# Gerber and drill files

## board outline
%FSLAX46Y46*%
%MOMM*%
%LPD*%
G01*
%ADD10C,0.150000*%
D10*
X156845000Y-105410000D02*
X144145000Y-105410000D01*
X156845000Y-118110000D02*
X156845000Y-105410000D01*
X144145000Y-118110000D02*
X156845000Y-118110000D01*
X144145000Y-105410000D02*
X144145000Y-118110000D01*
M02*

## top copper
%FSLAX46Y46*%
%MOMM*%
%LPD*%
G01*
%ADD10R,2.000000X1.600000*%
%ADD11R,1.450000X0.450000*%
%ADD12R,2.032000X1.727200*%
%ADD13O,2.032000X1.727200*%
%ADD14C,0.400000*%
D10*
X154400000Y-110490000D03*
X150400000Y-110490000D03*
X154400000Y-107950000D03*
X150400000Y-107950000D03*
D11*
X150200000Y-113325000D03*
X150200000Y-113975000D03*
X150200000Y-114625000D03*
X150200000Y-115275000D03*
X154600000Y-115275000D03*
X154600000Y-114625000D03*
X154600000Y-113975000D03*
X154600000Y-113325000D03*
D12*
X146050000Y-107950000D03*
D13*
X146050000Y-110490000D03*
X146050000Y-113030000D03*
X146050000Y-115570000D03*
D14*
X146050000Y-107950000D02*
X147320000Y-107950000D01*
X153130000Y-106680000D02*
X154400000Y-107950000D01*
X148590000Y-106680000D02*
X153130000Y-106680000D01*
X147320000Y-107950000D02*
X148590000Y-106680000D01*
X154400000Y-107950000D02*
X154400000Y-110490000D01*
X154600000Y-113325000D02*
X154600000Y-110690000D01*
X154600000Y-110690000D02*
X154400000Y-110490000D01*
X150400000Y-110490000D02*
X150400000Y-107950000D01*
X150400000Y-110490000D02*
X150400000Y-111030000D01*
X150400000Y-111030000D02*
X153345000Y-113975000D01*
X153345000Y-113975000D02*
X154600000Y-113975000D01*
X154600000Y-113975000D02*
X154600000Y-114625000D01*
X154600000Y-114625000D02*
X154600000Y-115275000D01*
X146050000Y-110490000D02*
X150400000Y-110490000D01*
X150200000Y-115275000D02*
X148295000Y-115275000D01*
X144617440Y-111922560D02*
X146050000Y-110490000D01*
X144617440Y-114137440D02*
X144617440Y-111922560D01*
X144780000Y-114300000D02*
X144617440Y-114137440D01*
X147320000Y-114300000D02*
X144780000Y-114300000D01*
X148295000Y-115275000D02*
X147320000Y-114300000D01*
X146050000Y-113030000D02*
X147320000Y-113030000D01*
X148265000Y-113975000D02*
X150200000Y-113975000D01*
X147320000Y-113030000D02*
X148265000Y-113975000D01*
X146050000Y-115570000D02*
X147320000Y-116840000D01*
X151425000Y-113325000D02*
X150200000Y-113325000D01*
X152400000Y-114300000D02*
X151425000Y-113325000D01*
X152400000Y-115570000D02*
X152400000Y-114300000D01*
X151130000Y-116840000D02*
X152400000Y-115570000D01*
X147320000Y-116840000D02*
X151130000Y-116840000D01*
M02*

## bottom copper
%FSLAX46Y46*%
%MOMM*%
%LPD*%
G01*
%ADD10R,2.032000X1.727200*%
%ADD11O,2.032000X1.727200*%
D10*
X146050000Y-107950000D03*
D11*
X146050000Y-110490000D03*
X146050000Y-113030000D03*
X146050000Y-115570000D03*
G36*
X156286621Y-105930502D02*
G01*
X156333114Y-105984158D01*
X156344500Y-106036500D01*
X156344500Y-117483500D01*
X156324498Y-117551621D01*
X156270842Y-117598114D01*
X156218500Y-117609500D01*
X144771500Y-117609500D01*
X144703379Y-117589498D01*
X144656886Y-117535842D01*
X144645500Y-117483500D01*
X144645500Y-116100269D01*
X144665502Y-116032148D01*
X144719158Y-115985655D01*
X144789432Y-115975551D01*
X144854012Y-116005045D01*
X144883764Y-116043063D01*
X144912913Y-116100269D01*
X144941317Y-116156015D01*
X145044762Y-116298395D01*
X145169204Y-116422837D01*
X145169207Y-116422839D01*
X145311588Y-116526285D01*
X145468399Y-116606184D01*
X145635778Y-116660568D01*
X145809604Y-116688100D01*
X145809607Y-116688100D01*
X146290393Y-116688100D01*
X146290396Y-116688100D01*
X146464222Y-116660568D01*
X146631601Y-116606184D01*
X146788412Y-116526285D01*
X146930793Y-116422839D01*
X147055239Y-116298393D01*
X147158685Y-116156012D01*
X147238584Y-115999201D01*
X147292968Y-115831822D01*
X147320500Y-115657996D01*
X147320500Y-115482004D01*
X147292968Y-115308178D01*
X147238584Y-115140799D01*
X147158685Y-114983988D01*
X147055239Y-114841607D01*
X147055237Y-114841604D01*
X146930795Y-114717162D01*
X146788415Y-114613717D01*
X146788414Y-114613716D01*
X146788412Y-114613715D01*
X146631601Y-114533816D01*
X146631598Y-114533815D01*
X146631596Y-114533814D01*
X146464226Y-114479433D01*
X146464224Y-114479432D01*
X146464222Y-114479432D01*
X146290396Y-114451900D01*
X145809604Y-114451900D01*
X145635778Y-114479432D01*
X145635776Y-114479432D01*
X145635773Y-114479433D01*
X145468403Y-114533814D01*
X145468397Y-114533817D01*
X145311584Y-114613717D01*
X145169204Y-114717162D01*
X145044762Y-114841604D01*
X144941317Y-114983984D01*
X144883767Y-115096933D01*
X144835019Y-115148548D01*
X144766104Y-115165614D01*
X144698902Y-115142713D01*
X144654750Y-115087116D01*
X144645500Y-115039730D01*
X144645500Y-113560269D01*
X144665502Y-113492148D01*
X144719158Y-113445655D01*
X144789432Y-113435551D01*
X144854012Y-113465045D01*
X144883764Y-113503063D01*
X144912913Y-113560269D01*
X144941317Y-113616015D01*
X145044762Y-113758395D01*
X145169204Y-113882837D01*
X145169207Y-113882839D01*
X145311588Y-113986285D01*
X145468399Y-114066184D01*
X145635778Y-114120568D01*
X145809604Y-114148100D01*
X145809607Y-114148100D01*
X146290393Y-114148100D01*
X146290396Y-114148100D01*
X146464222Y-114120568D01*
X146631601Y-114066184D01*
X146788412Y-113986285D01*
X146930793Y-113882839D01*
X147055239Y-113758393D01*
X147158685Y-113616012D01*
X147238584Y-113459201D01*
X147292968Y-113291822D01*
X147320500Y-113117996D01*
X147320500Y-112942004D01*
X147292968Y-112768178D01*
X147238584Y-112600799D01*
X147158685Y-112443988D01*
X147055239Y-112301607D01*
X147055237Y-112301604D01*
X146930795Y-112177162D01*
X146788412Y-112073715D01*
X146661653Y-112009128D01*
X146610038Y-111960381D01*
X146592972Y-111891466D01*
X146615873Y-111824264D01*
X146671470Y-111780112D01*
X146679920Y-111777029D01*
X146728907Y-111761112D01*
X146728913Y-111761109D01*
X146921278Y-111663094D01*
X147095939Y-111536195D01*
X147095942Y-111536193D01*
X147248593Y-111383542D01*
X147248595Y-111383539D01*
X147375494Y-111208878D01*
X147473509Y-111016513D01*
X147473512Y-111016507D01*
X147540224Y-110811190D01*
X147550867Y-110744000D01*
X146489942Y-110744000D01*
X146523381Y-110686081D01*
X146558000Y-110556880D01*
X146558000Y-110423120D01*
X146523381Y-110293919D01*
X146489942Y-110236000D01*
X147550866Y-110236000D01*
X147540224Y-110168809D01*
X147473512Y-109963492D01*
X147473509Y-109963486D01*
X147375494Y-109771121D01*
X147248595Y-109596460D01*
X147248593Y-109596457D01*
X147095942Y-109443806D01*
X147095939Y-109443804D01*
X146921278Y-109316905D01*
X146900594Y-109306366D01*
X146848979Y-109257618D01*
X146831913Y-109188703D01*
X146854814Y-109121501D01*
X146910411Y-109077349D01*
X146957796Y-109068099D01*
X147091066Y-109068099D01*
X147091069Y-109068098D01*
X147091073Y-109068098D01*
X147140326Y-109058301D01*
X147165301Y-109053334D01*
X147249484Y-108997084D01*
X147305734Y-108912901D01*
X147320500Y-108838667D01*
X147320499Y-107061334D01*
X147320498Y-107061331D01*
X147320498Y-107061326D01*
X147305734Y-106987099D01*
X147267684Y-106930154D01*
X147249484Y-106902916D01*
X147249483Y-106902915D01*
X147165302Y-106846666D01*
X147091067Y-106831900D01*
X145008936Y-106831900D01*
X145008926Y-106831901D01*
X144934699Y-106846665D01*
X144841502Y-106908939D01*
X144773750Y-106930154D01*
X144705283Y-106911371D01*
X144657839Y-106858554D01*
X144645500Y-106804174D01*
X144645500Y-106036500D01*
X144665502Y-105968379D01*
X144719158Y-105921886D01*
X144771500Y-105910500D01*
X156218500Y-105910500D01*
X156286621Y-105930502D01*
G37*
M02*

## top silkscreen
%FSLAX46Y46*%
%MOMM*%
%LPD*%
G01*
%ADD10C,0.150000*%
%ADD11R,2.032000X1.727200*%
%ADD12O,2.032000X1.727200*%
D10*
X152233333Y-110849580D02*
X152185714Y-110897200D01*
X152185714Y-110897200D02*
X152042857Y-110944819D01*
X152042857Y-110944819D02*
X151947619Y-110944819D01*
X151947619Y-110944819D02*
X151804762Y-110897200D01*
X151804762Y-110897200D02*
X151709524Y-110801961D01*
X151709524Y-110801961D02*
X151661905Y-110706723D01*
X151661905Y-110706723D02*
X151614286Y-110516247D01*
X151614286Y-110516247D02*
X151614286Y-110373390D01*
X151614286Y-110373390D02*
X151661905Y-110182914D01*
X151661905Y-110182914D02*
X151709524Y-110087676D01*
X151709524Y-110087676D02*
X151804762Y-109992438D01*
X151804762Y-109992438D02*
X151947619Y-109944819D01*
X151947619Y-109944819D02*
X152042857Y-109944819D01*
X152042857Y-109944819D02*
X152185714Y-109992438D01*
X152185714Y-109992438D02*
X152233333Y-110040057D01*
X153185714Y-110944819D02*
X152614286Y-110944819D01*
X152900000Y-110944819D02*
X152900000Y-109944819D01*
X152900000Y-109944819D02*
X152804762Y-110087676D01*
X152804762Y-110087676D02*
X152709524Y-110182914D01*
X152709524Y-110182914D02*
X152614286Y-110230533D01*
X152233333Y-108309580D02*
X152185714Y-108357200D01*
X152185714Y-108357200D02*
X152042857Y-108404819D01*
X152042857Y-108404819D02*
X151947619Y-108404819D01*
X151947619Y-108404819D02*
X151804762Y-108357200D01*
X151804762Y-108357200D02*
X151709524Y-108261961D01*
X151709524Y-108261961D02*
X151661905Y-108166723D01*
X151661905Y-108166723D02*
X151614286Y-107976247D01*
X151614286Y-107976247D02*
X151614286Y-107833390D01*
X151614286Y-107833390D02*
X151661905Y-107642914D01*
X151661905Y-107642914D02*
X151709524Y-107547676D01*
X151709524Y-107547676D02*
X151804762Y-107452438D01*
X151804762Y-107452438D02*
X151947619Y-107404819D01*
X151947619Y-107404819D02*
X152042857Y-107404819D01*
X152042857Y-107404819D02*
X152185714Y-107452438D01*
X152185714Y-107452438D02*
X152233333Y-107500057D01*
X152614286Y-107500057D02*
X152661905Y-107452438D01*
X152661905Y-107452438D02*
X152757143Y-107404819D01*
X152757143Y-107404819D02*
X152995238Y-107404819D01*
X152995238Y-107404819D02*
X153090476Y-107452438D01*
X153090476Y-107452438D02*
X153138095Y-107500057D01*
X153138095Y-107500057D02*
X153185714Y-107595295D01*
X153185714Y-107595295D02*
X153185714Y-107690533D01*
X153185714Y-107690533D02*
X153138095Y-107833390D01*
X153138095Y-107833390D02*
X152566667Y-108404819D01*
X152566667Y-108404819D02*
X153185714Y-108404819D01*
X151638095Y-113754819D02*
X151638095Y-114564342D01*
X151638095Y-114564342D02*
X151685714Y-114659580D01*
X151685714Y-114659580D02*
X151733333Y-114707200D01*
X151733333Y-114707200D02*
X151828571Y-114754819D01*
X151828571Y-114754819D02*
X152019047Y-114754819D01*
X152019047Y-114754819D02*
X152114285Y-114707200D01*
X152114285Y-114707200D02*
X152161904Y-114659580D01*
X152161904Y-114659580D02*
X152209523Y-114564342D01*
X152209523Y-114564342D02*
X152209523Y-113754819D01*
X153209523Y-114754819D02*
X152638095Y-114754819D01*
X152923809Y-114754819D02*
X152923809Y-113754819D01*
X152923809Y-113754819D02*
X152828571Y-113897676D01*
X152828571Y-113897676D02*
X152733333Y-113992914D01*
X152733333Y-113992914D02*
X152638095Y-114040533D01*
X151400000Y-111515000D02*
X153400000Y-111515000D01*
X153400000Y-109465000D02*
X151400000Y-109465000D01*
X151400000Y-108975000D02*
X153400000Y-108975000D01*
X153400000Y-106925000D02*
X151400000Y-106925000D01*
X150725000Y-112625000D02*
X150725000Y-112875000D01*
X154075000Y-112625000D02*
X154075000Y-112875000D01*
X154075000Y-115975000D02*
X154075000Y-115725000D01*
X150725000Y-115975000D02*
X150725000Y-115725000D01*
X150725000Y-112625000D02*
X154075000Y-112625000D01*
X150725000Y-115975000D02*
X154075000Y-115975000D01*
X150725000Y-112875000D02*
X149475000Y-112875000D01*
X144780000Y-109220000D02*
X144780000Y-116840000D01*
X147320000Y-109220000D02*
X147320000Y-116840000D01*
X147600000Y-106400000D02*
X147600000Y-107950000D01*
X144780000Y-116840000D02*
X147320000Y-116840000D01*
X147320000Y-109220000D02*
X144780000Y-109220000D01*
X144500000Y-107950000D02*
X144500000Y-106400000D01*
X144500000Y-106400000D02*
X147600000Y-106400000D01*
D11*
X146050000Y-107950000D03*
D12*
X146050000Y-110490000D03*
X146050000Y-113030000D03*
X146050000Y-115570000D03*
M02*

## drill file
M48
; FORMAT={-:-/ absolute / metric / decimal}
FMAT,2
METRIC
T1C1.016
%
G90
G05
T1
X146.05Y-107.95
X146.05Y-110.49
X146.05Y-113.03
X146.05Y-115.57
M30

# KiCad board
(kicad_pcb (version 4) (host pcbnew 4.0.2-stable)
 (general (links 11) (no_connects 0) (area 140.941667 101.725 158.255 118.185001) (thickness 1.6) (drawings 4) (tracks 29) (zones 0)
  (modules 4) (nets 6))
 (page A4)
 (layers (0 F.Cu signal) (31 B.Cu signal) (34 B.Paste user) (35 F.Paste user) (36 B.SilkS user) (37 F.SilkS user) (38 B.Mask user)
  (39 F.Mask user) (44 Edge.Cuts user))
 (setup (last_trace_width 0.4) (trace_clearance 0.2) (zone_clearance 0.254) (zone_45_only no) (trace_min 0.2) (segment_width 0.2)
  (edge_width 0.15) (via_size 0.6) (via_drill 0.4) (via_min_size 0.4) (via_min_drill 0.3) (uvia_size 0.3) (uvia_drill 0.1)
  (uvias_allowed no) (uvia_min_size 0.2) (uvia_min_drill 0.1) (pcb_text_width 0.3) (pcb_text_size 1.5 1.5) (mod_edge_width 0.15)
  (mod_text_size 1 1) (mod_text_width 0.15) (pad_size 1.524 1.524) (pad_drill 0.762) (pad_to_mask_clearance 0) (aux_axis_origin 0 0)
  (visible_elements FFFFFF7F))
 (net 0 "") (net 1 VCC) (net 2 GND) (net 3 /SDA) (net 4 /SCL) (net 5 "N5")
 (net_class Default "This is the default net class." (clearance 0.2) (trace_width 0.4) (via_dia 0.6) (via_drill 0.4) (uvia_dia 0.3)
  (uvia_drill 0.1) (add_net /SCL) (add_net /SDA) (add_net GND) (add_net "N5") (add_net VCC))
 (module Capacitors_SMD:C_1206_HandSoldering (layer F.Cu) (at 152.4 110.49 180)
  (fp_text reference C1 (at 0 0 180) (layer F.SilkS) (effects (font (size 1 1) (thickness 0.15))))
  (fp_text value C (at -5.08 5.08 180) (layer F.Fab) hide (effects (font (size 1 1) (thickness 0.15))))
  (fp_line (start 1 -1.025) (end -1 -1.025) (layer F.SilkS) (width 0.15))
  (fp_line (start -1 1.025) (end 1 1.025) (layer F.SilkS) (width 0.15))
  (pad 1 smd rect (at -2 0 180) (size 2 1.6) (layers F.Cu F.Paste F.Mask) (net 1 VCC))
  (pad 2 smd rect (at 2 0 180) (size 2 1.6) (layers F.Cu F.Paste F.Mask) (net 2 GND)))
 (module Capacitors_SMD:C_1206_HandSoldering (layer F.Cu) (at 152.4 107.95 180)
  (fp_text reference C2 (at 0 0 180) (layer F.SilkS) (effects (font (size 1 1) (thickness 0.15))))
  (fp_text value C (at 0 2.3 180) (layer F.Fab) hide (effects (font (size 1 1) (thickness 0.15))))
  (fp_line (start 1 -1.025) (end -1 -1.025) (layer F.SilkS) (width 0.15))
  (fp_line (start -1 1.025) (end 1 1.025) (layer F.SilkS) (width 0.15))
  (pad 1 smd rect (at -2 0 180) (size 2 1.6) (layers F.Cu F.Paste F.Mask) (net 1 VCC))
  (pad 2 smd rect (at 2 0 180) (size 2 1.6) (layers F.Cu F.Paste F.Mask) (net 2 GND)))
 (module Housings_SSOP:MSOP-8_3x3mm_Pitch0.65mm (layer F.Cu) (at 152.4 114.3)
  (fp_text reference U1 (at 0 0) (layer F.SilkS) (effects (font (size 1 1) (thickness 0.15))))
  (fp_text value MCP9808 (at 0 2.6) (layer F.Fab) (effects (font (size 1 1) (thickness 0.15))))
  (fp_line (start -1.675 -1.675) (end -1.675 -1.425) (layer F.SilkS) (width 0.15))
  (fp_line (start 1.675 -1.675) (end 1.675 -1.425) (layer F.SilkS) (width 0.15))
  (fp_line (start 1.675 1.675) (end 1.675 1.425) (layer F.SilkS) (width 0.15))
  (fp_line (start -1.675 1.675) (end -1.675 1.425) (layer F.SilkS) (width 0.15))
  (fp_line (start -1.675 -1.675) (end 1.675 -1.675) (layer F.SilkS) (width 0.15))
  (fp_line (start -1.675 1.675) (end 1.675 1.675) (layer F.SilkS) (width 0.15))
  (fp_line (start -1.675 -1.425) (end -2.925 -1.425) (layer F.SilkS) (width 0.15))
  (pad 1 smd rect (at -2.2 -0.975) (size 1.45 0.45) (layers F.Cu F.Paste F.Mask) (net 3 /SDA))
  (pad 2 smd rect (at -2.2 -0.325) (size 1.45 0.45) (layers F.Cu F.Paste F.Mask) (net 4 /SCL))
  (pad 3 smd rect (at -2.2 0.325) (size 1.45 0.45) (layers F.Cu F.Paste F.Mask) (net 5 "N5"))
  (pad 4 smd rect (at -2.2 0.975) (size 1.45 0.45) (layers F.Cu F.Paste F.Mask) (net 2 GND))
  (pad 5 smd rect (at 2.2 0.975) (size 1.45 0.45) (layers F.Cu F.Paste F.Mask) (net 2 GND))
  (pad 6 smd rect (at 2.2 0.325) (size 1.45 0.45) (layers F.Cu F.Paste F.Mask) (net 2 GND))
  (pad 7 smd rect (at 2.2 -0.325) (size 1.45 0.45) (layers F.Cu F.Paste F.Mask) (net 2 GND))
  (pad 8 smd rect (at 2.2 -0.975) (size 1.45 0.45) (layers F.Cu F.Paste F.Mask) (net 1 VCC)))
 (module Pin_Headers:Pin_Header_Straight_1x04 (layer F.Cu) (at 146.05 107.95)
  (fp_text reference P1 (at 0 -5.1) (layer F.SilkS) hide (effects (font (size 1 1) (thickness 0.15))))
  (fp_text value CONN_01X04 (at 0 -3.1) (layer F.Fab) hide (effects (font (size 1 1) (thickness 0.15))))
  (fp_line (start -1.27 1.27) (end -1.27 8.89) (layer F.SilkS) (width 0.15))
  (fp_line (start 1.27 1.27) (end 1.27 8.89) (layer F.SilkS) (width 0.15))
  (fp_line (start 1.55 -1.55) (end 1.55 0) (layer F.SilkS) (width 0.15))
  (fp_line (start -1.27 8.89) (end 1.27 8.89) (layer F.SilkS) (width 0.15))
  (fp_line (start 1.27 1.27) (end -1.27 1.27) (layer F.SilkS) (width 0.15))
  (fp_line (start -1.55 0) (end -1.55 -1.55) (layer F.SilkS) (width 0.15))
  (fp_line (start -1.55 -1.55) (end 1.55 -1.55) (layer F.SilkS) (width 0.15))
  (pad 1 thru_hole rect (at 0 0) (size 2.032 1.7272) (drill 1.016) (layers *.Cu *.Mask F.SilkS) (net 1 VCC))
  (pad 2 thru_hole oval (at 0 2.54) (size 2.032 1.7272) (drill 1.016) (layers *.Cu *.Mask F.SilkS) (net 2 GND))
  (pad 3 thru_hole oval (at 0 5.08) (size 2.032 1.7272) (drill 1.016) (layers *.Cu *.Mask F.SilkS) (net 4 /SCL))
  (pad 4 thru_hole oval (at 0 7.62) (size 2.032 1.7272) (drill 1.016) (layers *.Cu *.Mask F.SilkS) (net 3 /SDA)))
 (gr_line (start 156.845 105.41) (end 144.145 105.41) (angle 90) (layer Edge.Cuts) (width 0.15))
 (gr_line (start 156.845 118.11) (end 156.845 105.41) (angle 90) (layer Edge.Cuts) (width 0.15))
 (gr_line (start 144.145 118.11) (end 156.845 118.11) (angle 90) (layer Edge.Cuts) (width 0.15))
 (gr_line (start 144.145 105.41) (end 144.145 118.11) (angle 90) (layer Edge.Cuts) (width 0.15))
 (segment (start 146.05 107.95) (end 147.32 107.95) (width 0.4) (layer F.Cu) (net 1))
 (segment (start 153.13 106.68) (end 154.4 107.95) (width 0.4) (layer F.Cu) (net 1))
 (segment (start 148.59 106.68) (end 153.13 106.68) (width 0.4) (layer F.Cu) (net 1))
 (segment (start 147.32 107.95) (end 148.59 106.68) (width 0.4) (layer F.Cu) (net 1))
 (segment (start 154.4 107.95) (end 154.4 110.49) (width 0.4) (layer F.Cu) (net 1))
 (segment (start 154.6 113.325) (end 154.6 110.69) (width 0.4) (layer F.Cu) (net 1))
 (segment (start 154.6 110.69) (end 154.4 110.49) (width 0.4) (layer F.Cu) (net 1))
 (segment (start 150.4 110.49) (end 150.4 107.95) (width 0.4) (layer F.Cu) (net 2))
 (segment (start 150.4 110.49) (end 150.4 111.03) (width 0.4) (layer F.Cu) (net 2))
 (segment (start 150.4 111.03) (end 153.345 113.975) (width 0.4) (layer F.Cu) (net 2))
 (segment (start 153.345 113.975) (end 154.6 113.975) (width 0.4) (layer F.Cu) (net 2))
 (segment (start 154.6 113.975) (end 154.6 114.625) (width 0.4) (layer F.Cu) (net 2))
 (segment (start 154.6 114.625) (end 154.6 115.275) (width 0.4) (layer F.Cu) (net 2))
 (segment (start 146.05 110.49) (end 150.4 110.49) (width 0.4) (layer F.Cu) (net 2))
 (segment (start 150.2 115.275) (end 148.295 115.275) (width 0.4) (layer F.Cu) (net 2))
 (segment (start 144.61744 111.92256) (end 146.05 110.49) (width 0.4) (layer F.Cu) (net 2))
 (segment (start 144.61744 114.13744) (end 144.61744 111.92256) (width 0.4) (layer F.Cu) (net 2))
 (segment (start 144.78 114.3) (end 144.61744 114.13744) (width 0.4) (layer F.Cu) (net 2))
 (segment (start 147.32 114.3) (end 144.78 114.3) (width 0.4) (layer F.Cu) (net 2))
 (segment (start 148.295 115.275) (end 147.32 114.3) (width 0.4) (layer F.Cu) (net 2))
 (segment (start 146.05 113.03) (end 147.32 113.03) (width 0.4) (layer F.Cu) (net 4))
 (segment (start 148.265 113.975) (end 150.2 113.975) (width 0.4) (layer F.Cu) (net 4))
 (segment (start 147.32 113.03) (end 148.265 113.975) (width 0.4) (layer F.Cu) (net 4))
 (segment (start 146.05 115.57) (end 147.32 116.84) (width 0.4) (layer F.Cu) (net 3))
 (segment (start 151.425 113.325) (end 150.2 113.325) (width 0.4) (layer F.Cu) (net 3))
 (segment (start 152.4 114.3) (end 151.425 113.325) (width 0.4) (layer F.Cu) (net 3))
 (segment (start 152.4 115.57) (end 152.4 114.3) (width 0.4) (layer F.Cu) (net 3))
 (segment (start 151.13 116.84) (end 152.4 115.57) (width 0.4) (layer F.Cu) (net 3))
 (segment (start 147.32 116.84) (end 151.13 116.84) (width 0.4) (layer F.Cu) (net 3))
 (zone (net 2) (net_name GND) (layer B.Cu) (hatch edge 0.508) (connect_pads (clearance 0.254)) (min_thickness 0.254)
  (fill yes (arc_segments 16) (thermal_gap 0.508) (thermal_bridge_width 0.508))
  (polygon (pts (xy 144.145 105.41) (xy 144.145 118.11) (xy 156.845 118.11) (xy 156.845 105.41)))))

